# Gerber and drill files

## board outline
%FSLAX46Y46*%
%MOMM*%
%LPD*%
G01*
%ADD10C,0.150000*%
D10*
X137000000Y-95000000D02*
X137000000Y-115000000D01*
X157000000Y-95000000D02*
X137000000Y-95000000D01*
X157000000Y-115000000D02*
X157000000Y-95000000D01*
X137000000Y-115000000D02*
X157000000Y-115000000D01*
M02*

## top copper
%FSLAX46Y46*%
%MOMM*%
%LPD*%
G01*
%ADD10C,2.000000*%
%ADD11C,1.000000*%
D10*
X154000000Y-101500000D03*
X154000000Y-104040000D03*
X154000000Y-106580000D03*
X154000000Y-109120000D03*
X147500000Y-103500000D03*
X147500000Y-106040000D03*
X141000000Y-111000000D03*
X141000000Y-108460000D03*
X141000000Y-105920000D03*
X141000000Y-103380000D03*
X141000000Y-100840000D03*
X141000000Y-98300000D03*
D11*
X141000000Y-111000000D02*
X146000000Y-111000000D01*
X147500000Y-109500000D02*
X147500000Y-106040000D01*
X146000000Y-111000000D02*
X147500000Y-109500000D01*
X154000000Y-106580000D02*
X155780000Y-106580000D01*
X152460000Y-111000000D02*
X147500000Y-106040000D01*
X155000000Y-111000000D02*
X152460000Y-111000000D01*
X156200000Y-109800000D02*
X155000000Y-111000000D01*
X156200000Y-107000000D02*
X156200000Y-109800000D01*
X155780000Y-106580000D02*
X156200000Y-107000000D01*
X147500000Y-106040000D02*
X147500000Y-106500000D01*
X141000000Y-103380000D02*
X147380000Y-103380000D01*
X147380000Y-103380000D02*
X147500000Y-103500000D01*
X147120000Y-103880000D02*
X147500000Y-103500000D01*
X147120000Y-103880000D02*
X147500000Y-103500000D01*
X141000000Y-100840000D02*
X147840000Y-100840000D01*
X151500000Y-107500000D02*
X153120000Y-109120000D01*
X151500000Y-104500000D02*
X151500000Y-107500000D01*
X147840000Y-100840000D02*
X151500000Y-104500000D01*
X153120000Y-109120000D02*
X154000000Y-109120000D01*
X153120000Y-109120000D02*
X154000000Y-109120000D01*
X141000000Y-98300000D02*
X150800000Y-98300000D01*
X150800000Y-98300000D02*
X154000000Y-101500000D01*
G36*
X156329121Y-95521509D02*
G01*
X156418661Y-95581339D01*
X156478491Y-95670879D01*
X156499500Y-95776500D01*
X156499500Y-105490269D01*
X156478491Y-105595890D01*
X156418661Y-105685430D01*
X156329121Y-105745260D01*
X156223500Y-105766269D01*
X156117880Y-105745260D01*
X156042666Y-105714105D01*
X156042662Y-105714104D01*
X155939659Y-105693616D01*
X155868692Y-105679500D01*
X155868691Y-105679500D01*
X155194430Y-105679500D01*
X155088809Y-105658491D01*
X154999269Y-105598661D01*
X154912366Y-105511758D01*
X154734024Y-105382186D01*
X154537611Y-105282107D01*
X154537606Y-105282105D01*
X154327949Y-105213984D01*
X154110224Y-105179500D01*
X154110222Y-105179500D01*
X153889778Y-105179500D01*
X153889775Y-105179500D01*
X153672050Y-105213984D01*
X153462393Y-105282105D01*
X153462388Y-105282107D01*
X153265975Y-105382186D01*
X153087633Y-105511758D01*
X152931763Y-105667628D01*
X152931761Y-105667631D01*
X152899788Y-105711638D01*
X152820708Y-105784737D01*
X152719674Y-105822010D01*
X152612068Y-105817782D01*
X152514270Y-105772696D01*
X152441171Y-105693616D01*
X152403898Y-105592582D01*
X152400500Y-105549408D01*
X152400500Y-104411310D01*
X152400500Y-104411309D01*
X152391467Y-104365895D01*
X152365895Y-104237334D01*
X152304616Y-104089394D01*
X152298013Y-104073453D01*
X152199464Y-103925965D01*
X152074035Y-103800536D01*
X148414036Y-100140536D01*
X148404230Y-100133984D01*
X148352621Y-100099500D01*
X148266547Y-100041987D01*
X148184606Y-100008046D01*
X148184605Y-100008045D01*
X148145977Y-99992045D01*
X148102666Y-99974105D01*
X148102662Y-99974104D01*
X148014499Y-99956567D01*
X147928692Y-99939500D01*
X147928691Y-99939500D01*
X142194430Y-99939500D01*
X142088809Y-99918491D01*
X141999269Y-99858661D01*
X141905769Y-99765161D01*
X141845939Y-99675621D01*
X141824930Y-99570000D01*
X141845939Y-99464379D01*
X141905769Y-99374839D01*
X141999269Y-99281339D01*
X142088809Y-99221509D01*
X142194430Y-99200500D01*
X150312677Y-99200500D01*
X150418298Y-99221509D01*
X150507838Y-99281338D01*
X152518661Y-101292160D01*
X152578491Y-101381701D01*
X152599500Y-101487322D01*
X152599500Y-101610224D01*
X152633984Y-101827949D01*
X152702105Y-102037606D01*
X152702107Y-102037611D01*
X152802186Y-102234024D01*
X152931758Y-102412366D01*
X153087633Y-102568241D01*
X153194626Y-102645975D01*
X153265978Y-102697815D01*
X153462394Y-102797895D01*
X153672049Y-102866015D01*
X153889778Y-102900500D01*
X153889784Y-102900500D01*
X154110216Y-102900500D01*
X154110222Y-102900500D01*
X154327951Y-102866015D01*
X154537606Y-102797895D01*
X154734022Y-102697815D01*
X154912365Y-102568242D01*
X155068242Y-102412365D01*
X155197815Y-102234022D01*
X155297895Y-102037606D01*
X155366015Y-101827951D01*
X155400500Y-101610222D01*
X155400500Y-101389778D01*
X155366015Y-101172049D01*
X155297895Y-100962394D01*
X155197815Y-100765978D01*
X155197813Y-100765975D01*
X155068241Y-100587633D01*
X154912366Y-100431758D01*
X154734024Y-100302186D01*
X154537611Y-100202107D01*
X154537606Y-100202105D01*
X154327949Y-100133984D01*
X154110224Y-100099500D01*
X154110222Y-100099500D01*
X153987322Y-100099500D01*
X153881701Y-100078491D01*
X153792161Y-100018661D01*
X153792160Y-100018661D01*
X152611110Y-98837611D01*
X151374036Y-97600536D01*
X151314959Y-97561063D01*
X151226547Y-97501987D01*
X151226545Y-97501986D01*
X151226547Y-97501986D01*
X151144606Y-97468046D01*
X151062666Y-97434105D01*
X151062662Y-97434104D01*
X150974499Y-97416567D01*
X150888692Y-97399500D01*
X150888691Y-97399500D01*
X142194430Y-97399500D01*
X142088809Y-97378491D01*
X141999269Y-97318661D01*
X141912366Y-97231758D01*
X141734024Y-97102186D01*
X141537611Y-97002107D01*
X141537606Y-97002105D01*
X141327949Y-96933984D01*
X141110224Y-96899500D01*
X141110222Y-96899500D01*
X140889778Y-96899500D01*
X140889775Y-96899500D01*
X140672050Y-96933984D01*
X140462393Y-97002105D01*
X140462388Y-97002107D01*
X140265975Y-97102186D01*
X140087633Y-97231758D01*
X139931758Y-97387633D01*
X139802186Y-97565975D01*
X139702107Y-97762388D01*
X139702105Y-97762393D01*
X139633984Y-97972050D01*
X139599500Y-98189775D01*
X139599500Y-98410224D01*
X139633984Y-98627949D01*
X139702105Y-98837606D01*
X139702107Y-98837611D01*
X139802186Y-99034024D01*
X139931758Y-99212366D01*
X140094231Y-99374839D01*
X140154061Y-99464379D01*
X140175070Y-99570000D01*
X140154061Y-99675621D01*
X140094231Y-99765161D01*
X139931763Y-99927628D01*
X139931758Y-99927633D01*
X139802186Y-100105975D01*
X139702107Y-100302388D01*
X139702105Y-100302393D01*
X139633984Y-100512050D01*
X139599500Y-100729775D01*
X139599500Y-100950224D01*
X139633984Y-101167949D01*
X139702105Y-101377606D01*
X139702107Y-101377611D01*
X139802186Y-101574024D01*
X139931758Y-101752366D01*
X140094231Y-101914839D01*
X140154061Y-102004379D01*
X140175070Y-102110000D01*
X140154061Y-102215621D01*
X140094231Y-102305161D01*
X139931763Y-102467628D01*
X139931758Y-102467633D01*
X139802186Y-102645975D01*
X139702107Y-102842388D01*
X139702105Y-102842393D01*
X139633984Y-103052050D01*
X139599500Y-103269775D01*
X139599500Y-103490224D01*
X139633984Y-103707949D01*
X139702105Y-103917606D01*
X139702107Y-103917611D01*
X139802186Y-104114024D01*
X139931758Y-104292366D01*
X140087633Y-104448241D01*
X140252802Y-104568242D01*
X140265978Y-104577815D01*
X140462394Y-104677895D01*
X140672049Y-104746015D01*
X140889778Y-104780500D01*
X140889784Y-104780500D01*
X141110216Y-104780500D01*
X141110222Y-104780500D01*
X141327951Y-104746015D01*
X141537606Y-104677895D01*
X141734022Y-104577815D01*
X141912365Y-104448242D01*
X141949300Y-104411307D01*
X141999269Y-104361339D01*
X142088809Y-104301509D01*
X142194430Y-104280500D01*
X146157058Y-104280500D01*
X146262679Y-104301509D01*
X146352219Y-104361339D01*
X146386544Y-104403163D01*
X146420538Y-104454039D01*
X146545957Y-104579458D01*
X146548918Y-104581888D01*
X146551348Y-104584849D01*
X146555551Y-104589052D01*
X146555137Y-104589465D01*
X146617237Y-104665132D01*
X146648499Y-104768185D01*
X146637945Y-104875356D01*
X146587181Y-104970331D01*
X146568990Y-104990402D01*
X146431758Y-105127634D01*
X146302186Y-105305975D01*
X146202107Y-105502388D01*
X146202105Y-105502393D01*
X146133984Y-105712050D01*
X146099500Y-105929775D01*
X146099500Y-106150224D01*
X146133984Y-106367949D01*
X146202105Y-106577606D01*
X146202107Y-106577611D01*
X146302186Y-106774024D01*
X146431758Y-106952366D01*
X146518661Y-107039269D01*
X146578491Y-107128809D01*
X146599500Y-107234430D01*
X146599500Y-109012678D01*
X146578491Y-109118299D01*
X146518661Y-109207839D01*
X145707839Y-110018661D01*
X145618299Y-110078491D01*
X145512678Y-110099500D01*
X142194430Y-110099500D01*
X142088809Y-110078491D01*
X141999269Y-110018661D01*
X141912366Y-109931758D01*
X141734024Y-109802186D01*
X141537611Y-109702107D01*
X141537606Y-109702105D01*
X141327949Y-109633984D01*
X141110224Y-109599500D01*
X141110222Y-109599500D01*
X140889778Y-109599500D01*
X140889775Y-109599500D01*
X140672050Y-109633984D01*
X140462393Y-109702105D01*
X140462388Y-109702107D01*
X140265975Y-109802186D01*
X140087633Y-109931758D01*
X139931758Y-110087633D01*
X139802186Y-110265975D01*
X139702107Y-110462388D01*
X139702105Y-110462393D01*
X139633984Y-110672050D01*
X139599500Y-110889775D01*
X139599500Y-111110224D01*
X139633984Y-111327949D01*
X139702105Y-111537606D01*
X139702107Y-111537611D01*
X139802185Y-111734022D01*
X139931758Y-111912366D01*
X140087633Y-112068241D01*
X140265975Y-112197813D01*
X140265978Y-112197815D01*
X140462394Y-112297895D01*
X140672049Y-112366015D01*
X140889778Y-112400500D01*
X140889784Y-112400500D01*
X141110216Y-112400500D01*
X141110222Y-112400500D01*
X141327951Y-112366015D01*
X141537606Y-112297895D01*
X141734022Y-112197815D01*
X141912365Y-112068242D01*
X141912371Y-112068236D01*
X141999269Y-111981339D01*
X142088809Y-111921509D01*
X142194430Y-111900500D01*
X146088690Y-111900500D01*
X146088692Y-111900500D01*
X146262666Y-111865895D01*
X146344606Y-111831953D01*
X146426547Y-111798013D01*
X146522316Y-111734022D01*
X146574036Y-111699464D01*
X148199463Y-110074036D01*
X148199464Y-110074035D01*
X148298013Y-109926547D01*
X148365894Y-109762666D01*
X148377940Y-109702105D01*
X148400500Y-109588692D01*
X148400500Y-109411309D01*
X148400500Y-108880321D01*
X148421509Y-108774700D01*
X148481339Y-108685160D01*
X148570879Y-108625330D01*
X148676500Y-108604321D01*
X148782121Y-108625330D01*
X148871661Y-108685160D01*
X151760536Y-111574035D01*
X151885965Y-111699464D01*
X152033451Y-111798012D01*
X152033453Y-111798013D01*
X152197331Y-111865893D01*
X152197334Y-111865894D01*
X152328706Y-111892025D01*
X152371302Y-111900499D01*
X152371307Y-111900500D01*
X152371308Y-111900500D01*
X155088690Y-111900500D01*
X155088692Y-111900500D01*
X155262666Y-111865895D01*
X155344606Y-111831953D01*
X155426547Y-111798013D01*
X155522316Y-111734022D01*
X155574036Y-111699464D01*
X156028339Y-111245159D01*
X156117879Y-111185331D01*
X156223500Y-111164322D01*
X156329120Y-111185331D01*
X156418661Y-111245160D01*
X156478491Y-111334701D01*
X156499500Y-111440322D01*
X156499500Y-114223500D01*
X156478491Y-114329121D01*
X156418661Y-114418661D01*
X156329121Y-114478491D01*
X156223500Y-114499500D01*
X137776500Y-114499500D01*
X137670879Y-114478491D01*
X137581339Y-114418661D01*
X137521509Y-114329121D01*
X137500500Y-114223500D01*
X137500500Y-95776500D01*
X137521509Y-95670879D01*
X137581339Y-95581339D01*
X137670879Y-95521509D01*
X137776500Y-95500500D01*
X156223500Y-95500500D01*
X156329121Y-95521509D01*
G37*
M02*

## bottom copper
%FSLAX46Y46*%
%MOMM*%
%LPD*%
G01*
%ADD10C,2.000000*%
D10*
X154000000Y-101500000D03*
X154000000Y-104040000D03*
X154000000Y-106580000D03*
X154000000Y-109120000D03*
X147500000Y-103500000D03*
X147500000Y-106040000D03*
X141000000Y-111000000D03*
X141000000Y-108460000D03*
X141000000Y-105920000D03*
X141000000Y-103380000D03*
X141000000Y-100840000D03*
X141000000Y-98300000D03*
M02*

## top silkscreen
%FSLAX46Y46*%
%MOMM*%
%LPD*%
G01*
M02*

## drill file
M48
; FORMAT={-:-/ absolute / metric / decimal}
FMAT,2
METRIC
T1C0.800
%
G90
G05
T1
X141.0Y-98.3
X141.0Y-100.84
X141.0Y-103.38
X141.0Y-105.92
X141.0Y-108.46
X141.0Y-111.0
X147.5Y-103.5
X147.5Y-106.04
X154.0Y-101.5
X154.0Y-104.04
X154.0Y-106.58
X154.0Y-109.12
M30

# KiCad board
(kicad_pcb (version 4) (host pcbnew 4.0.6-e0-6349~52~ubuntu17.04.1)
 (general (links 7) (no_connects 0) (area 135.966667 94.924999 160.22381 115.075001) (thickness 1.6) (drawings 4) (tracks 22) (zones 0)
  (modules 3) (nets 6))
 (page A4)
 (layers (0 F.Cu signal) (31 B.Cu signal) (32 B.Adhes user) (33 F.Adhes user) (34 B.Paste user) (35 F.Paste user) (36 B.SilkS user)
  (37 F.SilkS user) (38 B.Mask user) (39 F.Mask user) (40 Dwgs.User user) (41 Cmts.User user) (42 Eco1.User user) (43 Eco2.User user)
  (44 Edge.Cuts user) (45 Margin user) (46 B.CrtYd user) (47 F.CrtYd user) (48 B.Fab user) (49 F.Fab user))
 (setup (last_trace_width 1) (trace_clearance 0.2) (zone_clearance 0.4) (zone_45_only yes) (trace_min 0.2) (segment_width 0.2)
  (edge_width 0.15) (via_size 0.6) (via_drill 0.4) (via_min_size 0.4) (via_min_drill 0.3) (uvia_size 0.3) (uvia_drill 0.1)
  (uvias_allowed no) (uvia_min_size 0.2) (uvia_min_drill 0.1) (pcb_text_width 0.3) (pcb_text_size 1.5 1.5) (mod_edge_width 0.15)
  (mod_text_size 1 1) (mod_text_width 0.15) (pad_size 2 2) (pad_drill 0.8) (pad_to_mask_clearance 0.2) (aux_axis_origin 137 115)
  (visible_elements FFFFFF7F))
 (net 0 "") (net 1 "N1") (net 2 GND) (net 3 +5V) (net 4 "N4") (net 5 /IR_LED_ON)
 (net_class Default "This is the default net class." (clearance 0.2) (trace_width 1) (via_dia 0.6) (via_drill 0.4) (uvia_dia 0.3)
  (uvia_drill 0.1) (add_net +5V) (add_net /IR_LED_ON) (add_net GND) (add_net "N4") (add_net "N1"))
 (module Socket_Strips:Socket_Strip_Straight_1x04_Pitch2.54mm (layer B.Cu) (at 154 101.5 180)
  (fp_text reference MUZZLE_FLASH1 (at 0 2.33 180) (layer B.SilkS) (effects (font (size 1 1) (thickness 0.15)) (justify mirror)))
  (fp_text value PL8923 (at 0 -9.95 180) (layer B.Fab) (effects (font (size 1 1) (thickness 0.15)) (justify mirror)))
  (pad 1 thru_hole circle (at 0 0 180) (size 2 2) (drill 0.8) (layers *.Cu *.Mask) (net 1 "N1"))
  (pad 2 thru_hole circle (at 0 -2.54 180) (size 2 2) (drill 0.8) (layers *.Cu *.Mask) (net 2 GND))
  (pad 3 thru_hole circle (at 0 -5.08 180) (size 2 2) (drill 0.8) (layers *.Cu *.Mask) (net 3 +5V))
  (pad 4 thru_hole circle (at 0 -7.62 180) (size 2 2) (drill 0.8) (layers *.Cu *.Mask) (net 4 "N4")))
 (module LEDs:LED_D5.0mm (layer B.Cu) (at 147.5 103.5 270)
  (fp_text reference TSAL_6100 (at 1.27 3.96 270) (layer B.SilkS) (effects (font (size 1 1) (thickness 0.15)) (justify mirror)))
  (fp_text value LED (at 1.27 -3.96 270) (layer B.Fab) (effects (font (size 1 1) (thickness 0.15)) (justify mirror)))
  (pad 1 thru_hole circle (at 0 0 270) (size 2 2) (drill 0.8) (layers *.Cu *.Mask) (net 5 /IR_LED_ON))
  (pad 2 thru_hole circle (at 2.54 0 270) (size 2 2) (drill 0.8) (layers *.Cu *.Mask) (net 3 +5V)))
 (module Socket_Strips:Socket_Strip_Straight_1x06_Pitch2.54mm (layer B.Cu) (at 141 111)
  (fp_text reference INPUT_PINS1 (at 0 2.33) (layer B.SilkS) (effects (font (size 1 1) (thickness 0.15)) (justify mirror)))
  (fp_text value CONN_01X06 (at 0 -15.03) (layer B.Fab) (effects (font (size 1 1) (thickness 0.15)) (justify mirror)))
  (pad 1 thru_hole circle (at 0 0) (size 2 2) (drill 0.8) (layers *.Cu *.Mask) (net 3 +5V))
  (pad 2 thru_hole circle (at 0 -2.54) (size 2 2) (drill 0.8) (layers *.Cu *.Mask) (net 2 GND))
  (pad 3 thru_hole circle (at 0 -5.08) (size 2 2) (drill 0.8) (layers *.Cu *.Mask) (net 2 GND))
  (pad 4 thru_hole circle (at 0 -7.62) (size 2 2) (drill 0.8) (layers *.Cu *.Mask) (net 5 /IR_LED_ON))
  (pad 5 thru_hole circle (at 0 -10.16) (size 2 2) (drill 0.8) (layers *.Cu *.Mask) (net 4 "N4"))
  (pad 6 thru_hole circle (at 0 -12.7) (size 2 2) (drill 0.8) (layers *.Cu *.Mask) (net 1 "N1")))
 (gr_line (start 137 95) (end 137 115) (angle 90) (layer Edge.Cuts) (width 0.15))
 (gr_line (start 157 95) (end 137 95) (angle 90) (layer Edge.Cuts) (width 0.15))
 (gr_line (start 157 115) (end 157 95) (angle 90) (layer Edge.Cuts) (width 0.15))
 (gr_line (start 137 115) (end 157 115) (angle 90) (layer Edge.Cuts) (width 0.15))
 (segment (start 141 111) (end 146 111) (width 1) (layer F.Cu) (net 3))
 (segment (start 147.5 109.5) (end 147.5 106.04) (width 1) (layer F.Cu) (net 3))
 (segment (start 146 111) (end 147.5 109.5) (width 1) (layer F.Cu) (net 3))
 (segment (start 154 106.58) (end 155.78 106.58) (width 1) (layer F.Cu) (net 3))
 (segment (start 152.46 111) (end 147.5 106.04) (width 1) (layer F.Cu) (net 3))
 (segment (start 155 111) (end 152.46 111) (width 1) (layer F.Cu) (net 3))
 (segment (start 156.2 109.8) (end 155 111) (width 1) (layer F.Cu) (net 3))
 (segment (start 156.2 107) (end 156.2 109.8) (width 1) (layer F.Cu) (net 3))
 (segment (start 155.78 106.58) (end 156.2 107) (width 1) (layer F.Cu) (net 3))
 (segment (start 147.5 106.04) (end 147.5 106.5) (width 1) (layer F.Cu) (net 3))
 (segment (start 141 103.38) (end 147.38 103.38) (width 1) (layer F.Cu) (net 5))
 (segment (start 147.38 103.38) (end 147.5 103.5) (width 1) (layer F.Cu) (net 5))
 (segment (start 147.12 103.88) (end 147.5 103.5) (width 1) (layer F.Cu) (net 5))
 (segment (start 147.12 103.88) (end 147.5 103.5) (width 1) (layer F.Cu) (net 5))
 (segment (start 141 100.84) (end 147.84 100.84) (width 1) (layer F.Cu) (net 4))
 (segment (start 151.5 107.5) (end 153.12 109.12) (width 1) (layer F.Cu) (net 4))
 (segment (start 151.5 104.5) (end 151.5 107.5) (width 1) (layer F.Cu) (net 4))
 (segment (start 147.84 100.84) (end 151.5 104.5) (width 1) (layer F.Cu) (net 4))
 (segment (start 153.12 109.12) (end 154 109.12) (width 1) (layer F.Cu) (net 4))
 (segment (start 153.12 109.12) (end 154 109.12) (width 1) (layer F.Cu) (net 4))
 (segment (start 141 98.3) (end 150.8 98.3) (width 1) (layer F.Cu) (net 1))
 (segment (start 150.8 98.3) (end 154 101.5) (width 1) (layer F.Cu) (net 1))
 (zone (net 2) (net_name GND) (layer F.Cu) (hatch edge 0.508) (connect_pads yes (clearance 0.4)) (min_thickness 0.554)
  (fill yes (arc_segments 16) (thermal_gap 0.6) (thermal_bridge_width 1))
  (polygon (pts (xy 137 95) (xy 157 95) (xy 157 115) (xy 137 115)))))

